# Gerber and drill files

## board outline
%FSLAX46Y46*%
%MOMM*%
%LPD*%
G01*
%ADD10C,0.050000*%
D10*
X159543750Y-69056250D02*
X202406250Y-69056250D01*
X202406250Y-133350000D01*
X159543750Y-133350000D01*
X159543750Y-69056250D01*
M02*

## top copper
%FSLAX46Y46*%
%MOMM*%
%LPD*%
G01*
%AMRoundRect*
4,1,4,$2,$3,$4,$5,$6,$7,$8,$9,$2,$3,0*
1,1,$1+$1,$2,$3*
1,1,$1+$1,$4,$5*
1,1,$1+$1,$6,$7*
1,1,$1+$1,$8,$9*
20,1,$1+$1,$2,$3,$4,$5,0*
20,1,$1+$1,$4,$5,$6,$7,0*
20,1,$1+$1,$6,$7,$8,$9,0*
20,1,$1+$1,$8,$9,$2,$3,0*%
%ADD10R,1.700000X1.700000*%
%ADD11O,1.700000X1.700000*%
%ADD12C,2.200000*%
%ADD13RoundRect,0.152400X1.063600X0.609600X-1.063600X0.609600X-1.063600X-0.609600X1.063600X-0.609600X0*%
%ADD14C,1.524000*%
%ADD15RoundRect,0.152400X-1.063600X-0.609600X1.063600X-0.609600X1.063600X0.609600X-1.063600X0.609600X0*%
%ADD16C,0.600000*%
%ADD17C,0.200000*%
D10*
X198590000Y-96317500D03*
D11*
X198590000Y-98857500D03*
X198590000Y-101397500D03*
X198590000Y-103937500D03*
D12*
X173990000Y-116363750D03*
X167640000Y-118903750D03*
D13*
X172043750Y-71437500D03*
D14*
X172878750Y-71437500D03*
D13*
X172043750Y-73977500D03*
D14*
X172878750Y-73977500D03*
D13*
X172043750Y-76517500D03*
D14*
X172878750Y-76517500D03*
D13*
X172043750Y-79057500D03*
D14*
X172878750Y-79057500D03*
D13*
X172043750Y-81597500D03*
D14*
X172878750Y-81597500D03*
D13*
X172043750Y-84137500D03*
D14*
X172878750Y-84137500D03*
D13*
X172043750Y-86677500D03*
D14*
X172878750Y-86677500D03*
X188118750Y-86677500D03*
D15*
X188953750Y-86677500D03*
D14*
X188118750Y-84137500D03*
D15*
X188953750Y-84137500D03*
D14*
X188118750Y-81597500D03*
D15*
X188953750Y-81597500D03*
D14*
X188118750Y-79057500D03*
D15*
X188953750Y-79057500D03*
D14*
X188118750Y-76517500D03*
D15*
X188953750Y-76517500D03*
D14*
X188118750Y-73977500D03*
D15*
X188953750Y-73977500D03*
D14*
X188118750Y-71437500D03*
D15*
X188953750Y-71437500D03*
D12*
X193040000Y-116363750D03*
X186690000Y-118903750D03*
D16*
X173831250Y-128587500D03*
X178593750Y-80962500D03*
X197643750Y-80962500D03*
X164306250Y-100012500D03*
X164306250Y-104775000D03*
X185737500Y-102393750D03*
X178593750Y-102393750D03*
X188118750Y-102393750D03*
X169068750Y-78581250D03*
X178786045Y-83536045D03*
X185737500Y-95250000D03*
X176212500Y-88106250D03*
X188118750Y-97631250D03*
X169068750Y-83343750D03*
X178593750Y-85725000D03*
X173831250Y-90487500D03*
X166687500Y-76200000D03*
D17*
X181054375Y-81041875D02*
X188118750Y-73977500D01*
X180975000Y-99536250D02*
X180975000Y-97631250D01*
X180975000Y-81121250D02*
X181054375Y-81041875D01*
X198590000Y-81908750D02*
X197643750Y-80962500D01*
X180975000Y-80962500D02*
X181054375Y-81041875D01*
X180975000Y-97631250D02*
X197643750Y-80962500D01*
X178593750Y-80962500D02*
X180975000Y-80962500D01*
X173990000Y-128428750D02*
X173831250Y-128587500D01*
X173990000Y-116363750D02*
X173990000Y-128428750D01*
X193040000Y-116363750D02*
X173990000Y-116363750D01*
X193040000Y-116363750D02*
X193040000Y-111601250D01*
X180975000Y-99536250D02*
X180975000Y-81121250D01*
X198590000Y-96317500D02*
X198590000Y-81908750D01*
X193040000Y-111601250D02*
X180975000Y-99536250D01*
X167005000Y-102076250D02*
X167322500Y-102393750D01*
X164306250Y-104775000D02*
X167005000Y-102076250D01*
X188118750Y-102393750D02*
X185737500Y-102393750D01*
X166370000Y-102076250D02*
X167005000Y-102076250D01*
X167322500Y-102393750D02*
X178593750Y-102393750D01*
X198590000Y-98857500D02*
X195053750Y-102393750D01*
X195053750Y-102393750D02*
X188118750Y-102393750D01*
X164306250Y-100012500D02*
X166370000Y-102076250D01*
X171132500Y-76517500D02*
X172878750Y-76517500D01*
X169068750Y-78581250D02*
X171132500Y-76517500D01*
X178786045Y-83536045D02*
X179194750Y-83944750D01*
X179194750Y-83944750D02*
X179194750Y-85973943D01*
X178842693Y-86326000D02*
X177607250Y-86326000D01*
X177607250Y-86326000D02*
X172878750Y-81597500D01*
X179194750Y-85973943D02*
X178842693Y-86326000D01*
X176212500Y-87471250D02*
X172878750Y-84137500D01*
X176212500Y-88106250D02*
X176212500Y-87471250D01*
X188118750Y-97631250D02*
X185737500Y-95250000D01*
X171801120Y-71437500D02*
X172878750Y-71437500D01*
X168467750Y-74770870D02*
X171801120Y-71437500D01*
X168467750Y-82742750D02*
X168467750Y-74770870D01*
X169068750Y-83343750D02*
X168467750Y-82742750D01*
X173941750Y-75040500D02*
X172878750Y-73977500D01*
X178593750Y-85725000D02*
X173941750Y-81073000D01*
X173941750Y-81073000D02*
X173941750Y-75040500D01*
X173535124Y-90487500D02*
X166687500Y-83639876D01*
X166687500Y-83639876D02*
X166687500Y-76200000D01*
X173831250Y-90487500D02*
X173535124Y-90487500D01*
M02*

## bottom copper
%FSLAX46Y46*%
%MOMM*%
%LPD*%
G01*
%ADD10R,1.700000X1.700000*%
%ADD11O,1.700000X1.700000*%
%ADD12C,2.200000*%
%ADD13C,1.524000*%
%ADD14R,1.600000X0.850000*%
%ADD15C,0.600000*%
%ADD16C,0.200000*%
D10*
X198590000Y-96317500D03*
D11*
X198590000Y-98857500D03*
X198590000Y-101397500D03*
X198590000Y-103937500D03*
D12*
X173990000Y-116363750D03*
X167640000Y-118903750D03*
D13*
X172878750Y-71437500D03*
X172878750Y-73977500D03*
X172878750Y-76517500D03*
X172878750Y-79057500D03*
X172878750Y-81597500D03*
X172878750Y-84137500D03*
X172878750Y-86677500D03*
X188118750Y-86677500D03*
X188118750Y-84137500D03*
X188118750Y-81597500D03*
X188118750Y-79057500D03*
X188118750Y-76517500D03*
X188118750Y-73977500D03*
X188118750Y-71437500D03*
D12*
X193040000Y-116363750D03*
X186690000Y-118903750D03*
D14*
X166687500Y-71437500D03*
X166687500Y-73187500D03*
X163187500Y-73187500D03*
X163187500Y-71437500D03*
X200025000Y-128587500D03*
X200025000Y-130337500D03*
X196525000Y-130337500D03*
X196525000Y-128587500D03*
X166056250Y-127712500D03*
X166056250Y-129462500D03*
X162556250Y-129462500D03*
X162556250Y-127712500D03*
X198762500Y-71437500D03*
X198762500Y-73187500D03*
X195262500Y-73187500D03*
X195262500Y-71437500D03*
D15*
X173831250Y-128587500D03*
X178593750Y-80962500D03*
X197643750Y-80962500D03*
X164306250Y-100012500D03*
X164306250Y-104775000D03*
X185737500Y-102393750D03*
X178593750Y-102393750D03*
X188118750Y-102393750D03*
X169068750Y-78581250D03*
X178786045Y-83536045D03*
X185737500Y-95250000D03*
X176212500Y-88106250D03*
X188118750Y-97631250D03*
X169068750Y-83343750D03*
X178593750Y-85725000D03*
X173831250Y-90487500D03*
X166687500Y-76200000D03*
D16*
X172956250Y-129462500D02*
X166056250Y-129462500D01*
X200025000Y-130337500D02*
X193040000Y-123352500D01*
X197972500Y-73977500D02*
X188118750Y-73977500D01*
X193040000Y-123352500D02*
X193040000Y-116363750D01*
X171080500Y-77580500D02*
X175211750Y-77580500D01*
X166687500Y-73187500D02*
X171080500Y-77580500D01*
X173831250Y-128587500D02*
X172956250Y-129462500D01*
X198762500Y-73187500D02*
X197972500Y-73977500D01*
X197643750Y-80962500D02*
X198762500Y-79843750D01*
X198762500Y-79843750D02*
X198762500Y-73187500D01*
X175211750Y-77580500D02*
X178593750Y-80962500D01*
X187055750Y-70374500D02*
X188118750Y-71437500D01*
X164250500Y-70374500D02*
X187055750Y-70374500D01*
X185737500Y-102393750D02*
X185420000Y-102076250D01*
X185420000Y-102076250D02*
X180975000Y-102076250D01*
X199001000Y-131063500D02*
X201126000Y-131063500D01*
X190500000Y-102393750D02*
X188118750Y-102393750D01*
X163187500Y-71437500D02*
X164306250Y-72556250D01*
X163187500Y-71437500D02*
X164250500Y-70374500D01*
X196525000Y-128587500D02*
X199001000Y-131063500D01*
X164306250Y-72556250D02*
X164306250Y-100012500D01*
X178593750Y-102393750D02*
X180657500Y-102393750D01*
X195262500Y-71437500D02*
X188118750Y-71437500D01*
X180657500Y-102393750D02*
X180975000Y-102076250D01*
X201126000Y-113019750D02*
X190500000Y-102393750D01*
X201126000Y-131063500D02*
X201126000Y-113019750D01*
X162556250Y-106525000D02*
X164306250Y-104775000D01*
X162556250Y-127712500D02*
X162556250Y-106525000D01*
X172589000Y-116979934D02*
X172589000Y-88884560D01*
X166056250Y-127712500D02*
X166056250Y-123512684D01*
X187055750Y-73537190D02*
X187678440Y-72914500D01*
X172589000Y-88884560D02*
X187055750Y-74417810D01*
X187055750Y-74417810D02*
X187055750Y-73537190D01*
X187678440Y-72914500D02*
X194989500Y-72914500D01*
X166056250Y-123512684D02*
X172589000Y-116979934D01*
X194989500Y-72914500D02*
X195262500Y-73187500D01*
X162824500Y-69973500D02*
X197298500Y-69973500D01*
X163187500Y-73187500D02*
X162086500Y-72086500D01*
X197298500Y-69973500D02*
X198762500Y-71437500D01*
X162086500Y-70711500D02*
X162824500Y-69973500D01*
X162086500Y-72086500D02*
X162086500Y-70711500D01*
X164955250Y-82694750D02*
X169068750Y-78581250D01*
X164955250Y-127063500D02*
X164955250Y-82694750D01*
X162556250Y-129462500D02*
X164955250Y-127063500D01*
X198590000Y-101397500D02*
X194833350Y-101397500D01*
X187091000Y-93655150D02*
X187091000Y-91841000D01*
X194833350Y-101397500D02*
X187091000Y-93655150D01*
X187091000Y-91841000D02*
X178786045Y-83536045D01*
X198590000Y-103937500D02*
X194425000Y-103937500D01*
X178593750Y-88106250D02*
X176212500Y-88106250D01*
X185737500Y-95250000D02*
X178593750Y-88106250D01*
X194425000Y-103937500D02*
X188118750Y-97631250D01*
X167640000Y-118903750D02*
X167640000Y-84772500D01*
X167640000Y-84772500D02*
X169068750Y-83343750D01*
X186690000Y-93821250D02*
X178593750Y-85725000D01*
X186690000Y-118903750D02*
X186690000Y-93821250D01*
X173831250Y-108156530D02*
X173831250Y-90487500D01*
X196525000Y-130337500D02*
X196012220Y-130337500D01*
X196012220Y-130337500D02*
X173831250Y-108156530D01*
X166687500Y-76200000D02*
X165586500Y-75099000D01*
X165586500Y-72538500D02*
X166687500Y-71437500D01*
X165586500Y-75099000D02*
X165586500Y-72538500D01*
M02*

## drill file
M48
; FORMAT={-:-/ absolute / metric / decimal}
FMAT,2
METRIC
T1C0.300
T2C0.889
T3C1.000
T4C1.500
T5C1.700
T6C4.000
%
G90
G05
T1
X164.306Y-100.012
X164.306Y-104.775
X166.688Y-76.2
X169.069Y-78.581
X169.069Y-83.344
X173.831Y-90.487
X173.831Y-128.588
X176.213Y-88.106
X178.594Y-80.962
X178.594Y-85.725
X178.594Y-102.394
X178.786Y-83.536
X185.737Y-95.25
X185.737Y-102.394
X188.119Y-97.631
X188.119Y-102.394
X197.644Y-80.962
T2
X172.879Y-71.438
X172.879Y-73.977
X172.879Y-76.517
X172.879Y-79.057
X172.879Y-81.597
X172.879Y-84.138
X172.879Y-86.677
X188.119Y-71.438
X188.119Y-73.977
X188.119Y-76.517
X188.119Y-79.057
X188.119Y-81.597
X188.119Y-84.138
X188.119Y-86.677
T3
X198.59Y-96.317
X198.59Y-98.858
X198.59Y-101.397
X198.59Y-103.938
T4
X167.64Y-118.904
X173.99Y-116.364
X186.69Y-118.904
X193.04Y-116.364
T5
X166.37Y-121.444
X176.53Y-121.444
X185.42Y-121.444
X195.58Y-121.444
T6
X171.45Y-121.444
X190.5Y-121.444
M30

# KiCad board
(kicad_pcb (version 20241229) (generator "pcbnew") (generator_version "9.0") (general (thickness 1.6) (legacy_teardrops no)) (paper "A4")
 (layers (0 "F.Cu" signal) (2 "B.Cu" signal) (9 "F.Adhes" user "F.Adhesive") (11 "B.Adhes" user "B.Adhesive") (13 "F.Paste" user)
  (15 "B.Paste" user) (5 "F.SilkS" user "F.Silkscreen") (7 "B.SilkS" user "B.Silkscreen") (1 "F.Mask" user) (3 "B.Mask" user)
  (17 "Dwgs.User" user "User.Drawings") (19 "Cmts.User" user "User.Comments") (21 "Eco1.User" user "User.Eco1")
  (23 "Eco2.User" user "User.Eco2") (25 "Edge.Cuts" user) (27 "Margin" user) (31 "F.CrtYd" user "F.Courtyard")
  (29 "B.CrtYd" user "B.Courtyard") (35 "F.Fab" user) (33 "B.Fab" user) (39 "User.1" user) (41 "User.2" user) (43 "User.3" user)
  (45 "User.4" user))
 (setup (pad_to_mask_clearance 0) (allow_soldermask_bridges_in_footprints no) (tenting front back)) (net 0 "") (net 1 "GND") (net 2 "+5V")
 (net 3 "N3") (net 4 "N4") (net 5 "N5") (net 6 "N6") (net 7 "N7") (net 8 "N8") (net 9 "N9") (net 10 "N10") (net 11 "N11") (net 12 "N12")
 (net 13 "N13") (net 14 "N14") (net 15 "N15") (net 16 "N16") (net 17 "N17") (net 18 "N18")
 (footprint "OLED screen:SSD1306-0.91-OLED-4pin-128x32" (layer "F.Cu") (at 162.09 94.1275)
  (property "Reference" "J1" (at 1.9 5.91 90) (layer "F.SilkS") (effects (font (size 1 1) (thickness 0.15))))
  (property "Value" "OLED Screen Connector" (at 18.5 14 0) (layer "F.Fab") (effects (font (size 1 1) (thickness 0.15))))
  (pad "1" thru_hole rect (at 36.5 2.19) (size 1.7 1.7) (drill 1) (layers "*.Cu" "*.Mask") (remove_unused_layers no) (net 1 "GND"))
  (pad "2" thru_hole oval (at 36.5 4.73) (size 1.7 1.7) (drill 1) (layers "*.Cu" "*.Mask") (remove_unused_layers no) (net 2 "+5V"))
  (pad "3" thru_hole oval (at 36.5 7.27) (size 1.7 1.7) (drill 1) (layers "*.Cu" "*.Mask") (remove_unused_layers no) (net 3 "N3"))
  (pad "4" thru_hole oval (at 36.5 9.81) (size 1.7 1.7) (drill 1) (layers "*.Cu" "*.Mask") (remove_unused_layers no) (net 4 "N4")))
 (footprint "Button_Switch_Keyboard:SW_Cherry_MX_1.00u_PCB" (layer "F.Cu") (at 173.99 116.36375)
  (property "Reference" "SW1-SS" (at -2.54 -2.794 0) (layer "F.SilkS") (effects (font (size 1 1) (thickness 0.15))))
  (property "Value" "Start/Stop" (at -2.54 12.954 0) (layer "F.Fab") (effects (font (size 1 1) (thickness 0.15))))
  (pad "" np_thru_hole circle (at -7.62 5.08) (size 1.7 1.7) (drill 1.7) (layers "*.Cu" "*.Mask"))
  (pad "" np_thru_hole circle (at -2.54 5.08) (size 4 4) (drill 4) (layers "*.Cu" "*.Mask"))
  (pad "" np_thru_hole circle (at 2.54 5.08) (size 1.7 1.7) (drill 1.7) (layers "*.Cu" "*.Mask"))
  (pad "1" thru_hole circle (at 0 0) (size 2.2 2.2) (drill 1.5) (layers "*.Cu" "*.Mask") (remove_unused_layers no) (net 1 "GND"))
  (pad "2" thru_hole circle (at -6.35 2.54) (size 2.2 2.2) (drill 1.5) (layers "*.Cu" "*.Mask") (remove_unused_layers no) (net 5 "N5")))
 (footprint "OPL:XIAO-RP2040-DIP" (layer "F.Cu") (at 180.49875 79.0575)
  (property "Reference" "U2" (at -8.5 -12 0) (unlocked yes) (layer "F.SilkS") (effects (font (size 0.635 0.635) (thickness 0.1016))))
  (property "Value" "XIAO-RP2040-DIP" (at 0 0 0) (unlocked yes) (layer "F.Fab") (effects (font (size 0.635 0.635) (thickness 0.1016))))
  (pad "1" smd roundrect (at -8.455 -7.62 180) (size 2.432 1.524) (layers "F.Cu" "F.Mask") (roundrect_rratio 0.1) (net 5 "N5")
   (thermal_bridge_angle 45))
  (pad "1" thru_hole circle (at -7.62 -7.62 180) (size 1.524 1.524) (drill 0.889) (layers "*.Cu" "*.Mask") (remove_unused_layers no)
   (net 5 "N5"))
  (pad "2" smd roundrect (at -8.455 -5.08 180) (size 2.432 1.524) (layers "F.Cu" "F.Mask") (roundrect_rratio 0.1) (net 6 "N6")
   (thermal_bridge_angle 45))
  (pad "2" thru_hole circle (at -7.62 -5.08 180) (size 1.524 1.524) (drill 0.889) (layers "*.Cu" "*.Mask") (remove_unused_layers no)
   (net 6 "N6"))
  (pad "3" smd roundrect (at -8.455 -2.54 180) (size 2.432 1.524) (layers "F.Cu" "F.Mask") (roundrect_rratio 0.1) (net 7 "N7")
   (thermal_bridge_angle 45))
  (pad "3" thru_hole circle (at -7.62 -2.54 180) (size 1.524 1.524) (drill 0.889) (layers "*.Cu" "*.Mask") (remove_unused_layers no)
   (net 7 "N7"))
  (pad "4" smd roundrect (at -8.455 0 180) (size 2.432 1.524) (layers "F.Cu" "F.Mask") (roundrect_rratio 0.1) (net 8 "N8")
   (thermal_bridge_angle 45))
  (pad "4" thru_hole circle (at -7.62 0 180) (size 1.524 1.524) (drill 0.889) (layers "*.Cu" "*.Mask") (remove_unused_layers no)
   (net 8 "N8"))
  (pad "5" smd roundrect (at -8.455 2.54 180) (size 2.432 1.524) (layers "F.Cu" "F.Mask") (roundrect_rratio 0.1) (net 3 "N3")
   (thermal_bridge_angle 45))
  (pad "5" thru_hole circle (at -7.62 2.54 180) (size 1.524 1.524) (drill 0.889) (layers "*.Cu" "*.Mask") (remove_unused_layers no)
   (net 3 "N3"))
  (pad "6" smd roundrect (at -8.455 5.08 180) (size 2.432 1.524) (layers "F.Cu" "F.Mask") (roundrect_rratio 0.1) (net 4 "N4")
   (thermal_bridge_angle 45))
  (pad "6" thru_hole circle (at -7.62 5.08 180) (size 1.524 1.524) (drill 0.889) (layers "*.Cu" "*.Mask") (remove_unused_layers no)
   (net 4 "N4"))
  (pad "7" smd roundrect (at -8.455 7.62 180) (size 2.432 1.524) (layers "F.Cu" "F.Mask") (roundrect_rratio 0.1) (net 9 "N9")
   (thermal_bridge_angle 45))
  (pad "7" thru_hole circle (at -7.62 7.62 180) (size 1.524 1.524) (drill 0.889) (layers "*.Cu" "*.Mask") (remove_unused_layers no)
   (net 9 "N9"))
  (pad "8" thru_hole circle (at 7.62 7.62) (size 1.524 1.524) (drill 0.889) (layers "*.Cu" "*.Mask") (remove_unused_layers no)
   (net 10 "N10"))
  (pad "8" smd roundrect (at 8.455 7.62) (size 2.432 1.524) (layers "F.Cu" "F.Mask") (roundrect_rratio 0.1) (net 10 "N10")
   (thermal_bridge_angle 45))
  (pad "9" thru_hole circle (at 7.62 5.08) (size 1.524 1.524) (drill 0.889) (layers "*.Cu" "*.Mask") (remove_unused_layers no)
   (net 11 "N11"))
  (pad "9" smd roundrect (at 8.455 5.08) (size 2.432 1.524) (layers "F.Cu" "F.Mask") (roundrect_rratio 0.1) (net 11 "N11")
   (thermal_bridge_angle 45))
  (pad "10" thru_hole circle (at 7.62 2.54) (size 1.524 1.524) (drill 0.889) (layers "*.Cu" "*.Mask") (remove_unused_layers no)
   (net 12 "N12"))
  (pad "10" smd roundrect (at 8.455 2.54) (size 2.432 1.524) (layers "F.Cu" "F.Mask") (roundrect_rratio 0.1) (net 12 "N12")
   (thermal_bridge_angle 45))
  (pad "11" thru_hole circle (at 7.62 0) (size 1.524 1.524) (drill 0.889) (layers "*.Cu" "*.Mask") (remove_unused_layers no) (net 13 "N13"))
  (pad "11" smd roundrect (at 8.455 0) (size 2.432 1.524) (layers "F.Cu" "F.Mask") (roundrect_rratio 0.1) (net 13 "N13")
   (thermal_bridge_angle 45))
  (pad "12" thru_hole circle (at 7.62 -2.54) (size 1.524 1.524) (drill 0.889) (layers "*.Cu" "*.Mask") (remove_unused_layers no)
   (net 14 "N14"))
  (pad "12" smd roundrect (at 8.455 -2.54) (size 2.432 1.524) (layers "F.Cu" "F.Mask") (roundrect_rratio 0.1) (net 14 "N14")
   (thermal_bridge_angle 45))
  (pad "13" thru_hole circle (at 7.62 -5.08) (size 1.524 1.524) (drill 0.889) (layers "*.Cu" "*.Mask") (remove_unused_layers no)
   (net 1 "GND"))
  (pad "13" smd roundrect (at 8.455 -5.08) (size 2.432 1.524) (layers "F.Cu" "F.Mask") (roundrect_rratio 0.1) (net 1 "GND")
   (thermal_bridge_angle 45))
  (pad "14" thru_hole circle (at 7.62 -7.62) (size 1.524 1.524) (drill 0.889) (layers "*.Cu" "*.Mask") (remove_unused_layers no)
   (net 2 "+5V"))
  (pad "14" smd roundrect (at 8.455 -7.62) (size 2.432 1.524) (layers "F.Cu" "F.Mask") (roundrect_rratio 0.1) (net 2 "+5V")
   (thermal_bridge_angle 45)))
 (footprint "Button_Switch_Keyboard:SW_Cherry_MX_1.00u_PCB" (layer "F.Cu") (at 193.04 116.36375)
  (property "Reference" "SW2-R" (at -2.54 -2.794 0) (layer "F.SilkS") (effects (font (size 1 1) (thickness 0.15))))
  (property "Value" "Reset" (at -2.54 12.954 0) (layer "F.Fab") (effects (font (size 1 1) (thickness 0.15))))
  (pad "" np_thru_hole circle (at -7.62 5.08) (size 1.7 1.7) (drill 1.7) (layers "*.Cu" "*.Mask"))
  (pad "" np_thru_hole circle (at -2.54 5.08) (size 4 4) (drill 4) (layers "*.Cu" "*.Mask"))
  (pad "" np_thru_hole circle (at 2.54 5.08) (size 1.7 1.7) (drill 1.7) (layers "*.Cu" "*.Mask"))
  (pad "1" thru_hole circle (at 0 0) (size 2.2 2.2) (drill 1.5) (layers "*.Cu" "*.Mask") (remove_unused_layers no) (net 1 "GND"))
  (pad "2" thru_hole circle (at -6.35 2.54) (size 2.2 2.2) (drill 1.5) (layers "*.Cu" "*.Mask") (remove_unused_layers no) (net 6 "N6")))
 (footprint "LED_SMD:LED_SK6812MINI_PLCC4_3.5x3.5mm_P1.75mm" (layer "B.Cu") (at 164.9375 72.3125 180)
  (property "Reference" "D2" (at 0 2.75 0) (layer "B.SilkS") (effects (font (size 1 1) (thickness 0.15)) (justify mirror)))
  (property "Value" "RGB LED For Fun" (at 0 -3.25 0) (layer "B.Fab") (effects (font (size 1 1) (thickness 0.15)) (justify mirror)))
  (pad "1" smd rect (at -1.75 0.875 180) (size 1.6 0.85) (layers "B.Cu" "B.Mask" "B.Paste") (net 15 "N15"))
  (pad "2" smd rect (at -1.75 -0.875 180) (size 1.6 0.85) (layers "B.Cu" "B.Mask" "B.Paste") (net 1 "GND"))
  (pad "3" smd rect (at 1.75 -0.875 180) (size 1.6 0.85) (layers "B.Cu" "B.Mask" "B.Paste") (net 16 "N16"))
  (pad "4" smd rect (at 1.75 0.875 180) (size 1.6 0.85) (layers "B.Cu" "B.Mask" "B.Paste") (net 2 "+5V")))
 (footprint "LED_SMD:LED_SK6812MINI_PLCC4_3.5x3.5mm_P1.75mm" (layer "B.Cu") (at 198.275 129.4625 180)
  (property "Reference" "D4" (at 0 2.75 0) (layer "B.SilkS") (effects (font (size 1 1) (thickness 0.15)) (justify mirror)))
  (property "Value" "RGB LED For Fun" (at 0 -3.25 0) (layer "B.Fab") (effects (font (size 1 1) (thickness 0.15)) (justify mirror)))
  (pad "1" smd rect (at -1.75 0.875 180) (size 1.6 0.85) (layers "B.Cu" "B.Mask" "B.Paste") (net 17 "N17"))
  (pad "2" smd rect (at -1.75 -0.875 180) (size 1.6 0.85) (layers "B.Cu" "B.Mask" "B.Paste") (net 1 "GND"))
  (pad "3" smd rect (at 1.75 -0.875 180) (size 1.6 0.85) (layers "B.Cu" "B.Mask" "B.Paste") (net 15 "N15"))
  (pad "4" smd rect (at 1.75 0.875 180) (size 1.6 0.85) (layers "B.Cu" "B.Mask" "B.Paste") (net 2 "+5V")))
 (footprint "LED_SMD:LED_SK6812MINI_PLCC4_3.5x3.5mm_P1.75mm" (layer "B.Cu") (at 164.30625 128.5875 180)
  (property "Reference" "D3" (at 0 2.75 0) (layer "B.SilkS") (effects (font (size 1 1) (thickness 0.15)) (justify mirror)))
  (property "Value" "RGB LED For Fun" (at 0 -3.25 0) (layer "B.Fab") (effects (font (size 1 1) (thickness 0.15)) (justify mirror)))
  (pad "1" smd rect (at -1.75 0.875 180) (size 1.6 0.85) (layers "B.Cu" "B.Mask" "B.Paste") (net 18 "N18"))
  (pad "2" smd rect (at -1.75 -0.875 180) (size 1.6 0.85) (layers "B.Cu" "B.Mask" "B.Paste") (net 1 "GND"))
  (pad "3" smd rect (at 1.75 -0.875 180) (size 1.6 0.85) (layers "B.Cu" "B.Mask" "B.Paste") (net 7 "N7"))
  (pad "4" smd rect (at 1.75 0.875 180) (size 1.6 0.85) (layers "B.Cu" "B.Mask" "B.Paste") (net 2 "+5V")))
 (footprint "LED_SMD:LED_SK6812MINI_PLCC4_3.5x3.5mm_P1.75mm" (layer "B.Cu") (at 197.0125 72.3125 180)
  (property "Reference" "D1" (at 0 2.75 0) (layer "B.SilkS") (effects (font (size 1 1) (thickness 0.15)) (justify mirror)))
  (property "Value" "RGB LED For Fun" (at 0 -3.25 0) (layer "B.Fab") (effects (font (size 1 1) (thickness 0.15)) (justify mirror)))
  (pad "1" smd rect (at -1.75 0.875 180) (size 1.6 0.85) (layers "B.Cu" "B.Mask" "B.Paste") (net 16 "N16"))
  (pad "2" smd rect (at -1.75 -0.875 180) (size 1.6 0.85) (layers "B.Cu" "B.Mask" "B.Paste") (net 1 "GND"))
  (pad "3" smd rect (at 1.75 -0.875 180) (size 1.6 0.85) (layers "B.Cu" "B.Mask" "B.Paste") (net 18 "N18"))
  (pad "4" smd rect (at 1.75 0.875 180) (size 1.6 0.85) (layers "B.Cu" "B.Mask" "B.Paste") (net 2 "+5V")))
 (gr_rect (start 159.54375 69.05625) (end 202.40625 133.35) (stroke (width 0.05) (type default)) (fill no) (layer "Edge.Cuts"))
 (segment (start 181.054375 81.041875) (end 188.11875 73.9775) (width 0.2) (layer "F.Cu") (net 1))
 (segment (start 180.975 99.53625) (end 180.975 97.63125) (width 0.2) (layer "F.Cu") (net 1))
 (segment (start 180.975 81.12125) (end 181.054375 81.041875) (width 0.2) (layer "F.Cu") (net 1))
 (segment (start 198.59 81.90875) (end 197.64375 80.9625) (width 0.2) (layer "F.Cu") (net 1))
 (segment (start 180.975 80.9625) (end 181.054375 81.041875) (width 0.2) (layer "F.Cu") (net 1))
 (segment (start 180.975 97.63125) (end 197.64375 80.9625) (width 0.2) (layer "F.Cu") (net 1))
 (segment (start 178.59375 80.9625) (end 180.975 80.9625) (width 0.2) (layer "F.Cu") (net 1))
 (segment (start 173.99 128.42875) (end 173.83125 128.5875) (width 0.2) (layer "F.Cu") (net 1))
 (segment (start 173.99 116.36375) (end 173.99 128.42875) (width 0.2) (layer "F.Cu") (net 1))
 (segment (start 193.04 116.36375) (end 173.99 116.36375) (width 0.2) (layer "F.Cu") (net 1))
 (segment (start 193.04 116.36375) (end 193.04 111.60125) (width 0.2) (layer "F.Cu") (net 1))
 (segment (start 180.975 99.53625) (end 180.975 81.12125) (width 0.2) (layer "F.Cu") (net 1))
 (segment (start 198.59 96.3175) (end 198.59 81.90875) (width 0.2) (layer "F.Cu") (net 1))
 (segment (start 193.04 111.60125) (end 180.975 99.53625) (width 0.2) (layer "F.Cu") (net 1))
 (via (at 173.83125 128.5875) (size 0.6) (drill 0.3) (layers "F.Cu" "B.Cu") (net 1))
 (via (at 178.59375 80.9625) (size 0.6) (drill 0.3) (layers "F.Cu" "B.Cu") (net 1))
 (via (at 197.64375 80.9625) (size 0.6) (drill 0.3) (layers "F.Cu" "B.Cu") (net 1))
 (segment (start 172.95625 129.4625) (end 166.05625 129.4625) (width 0.2) (layer "B.Cu") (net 1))
 (segment (start 200.025 130.3375) (end 193.04 123.3525) (width 0.2) (layer "B.Cu") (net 1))
 (segment (start 197.9725 73.9775) (end 188.11875 73.9775) (width 0.2) (layer "B.Cu") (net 1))
 (segment (start 193.04 123.3525) (end 193.04 116.36375) (width 0.2) (layer "B.Cu") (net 1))
 (segment (start 171.0805 77.5805) (end 175.21175 77.5805) (width 0.2) (layer "B.Cu") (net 1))
 (segment (start 166.6875 73.1875) (end 171.0805 77.5805) (width 0.2) (layer "B.Cu") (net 1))
 (segment (start 173.83125 128.5875) (end 172.95625 129.4625) (width 0.2) (layer "B.Cu") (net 1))
 (segment (start 198.7625 73.1875) (end 197.9725 73.9775) (width 0.2) (layer "B.Cu") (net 1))
 (segment (start 197.64375 80.9625) (end 198.7625 79.84375) (width 0.2) (layer "B.Cu") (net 1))
 (segment (start 198.7625 79.84375) (end 198.7625 73.1875) (width 0.2) (layer "B.Cu") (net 1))
 (segment (start 175.21175 77.5805) (end 178.59375 80.9625) (width 0.2) (layer "B.Cu") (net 1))
 (segment (start 167.005 102.07625) (end 167.3225 102.39375) (width 0.2) (layer "F.Cu") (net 2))
 (segment (start 164.30625 104.775) (end 167.005 102.07625) (width 0.2) (layer "F.Cu") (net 2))
 (segment (start 188.11875 102.39375) (end 185.7375 102.39375) (width 0.2) (layer "F.Cu") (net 2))
 (segment (start 166.37 102.07625) (end 167.005 102.07625) (width 0.2) (layer "F.Cu") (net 2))
 (segment (start 167.3225 102.39375) (end 178.59375 102.39375) (width 0.2) (layer "F.Cu") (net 2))
 (segment (start 198.59 98.8575) (end 195.05375 102.39375) (width 0.2) (layer "F.Cu") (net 2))
 (segment (start 195.05375 102.39375) (end 188.11875 102.39375) (width 0.2) (layer "F.Cu") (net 2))
 (segment (start 164.30625 100.0125) (end 166.37 102.07625) (width 0.2) (layer "F.Cu") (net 2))
 (via (at 164.30625 100.0125) (size 0.6) (drill 0.3) (layers "F.Cu" "B.Cu") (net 2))
 (via (at 164.30625 104.775) (size 0.6) (drill 0.3) (layers "F.Cu" "B.Cu") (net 2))
 (via (at 185.7375 102.39375) (size 0.6) (drill 0.3) (layers "F.Cu" "B.Cu") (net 2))
 (via (at 178.59375 102.39375) (size 0.6) (drill 0.3) (layers "F.Cu" "B.Cu") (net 2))
 (via (at 188.11875 102.39375) (size 0.6) (drill 0.3) (layers "F.Cu" "B.Cu") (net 2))
 (segment (start 187.05575 70.3745) (end 188.11875 71.4375) (width 0.2) (layer "B.Cu") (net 2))
 (segment (start 164.2505 70.3745) (end 187.05575 70.3745) (width 0.2) (layer "B.Cu") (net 2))
 (segment (start 185.7375 102.39375) (end 185.42 102.07625) (width 0.2) (layer "B.Cu") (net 2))
 (segment (start 185.42 102.07625) (end 180.975 102.07625) (width 0.2) (layer "B.Cu") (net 2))
 (segment (start 199.001 131.0635) (end 201.126 131.0635) (width 0.2) (layer "B.Cu") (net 2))
 (segment (start 190.5 102.39375) (end 188.11875 102.39375) (width 0.2) (layer "B.Cu") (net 2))
 (segment (start 163.1875 71.4375) (end 164.30625 72.55625) (width 0.2) (layer "B.Cu") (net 2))
 (segment (start 163.1875 71.4375) (end 164.2505 70.3745) (width 0.2) (layer "B.Cu") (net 2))
 (segment (start 196.525 128.5875) (end 199.001 131.0635) (width 0.2) (layer "B.Cu") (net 2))
 (segment (start 164.30625 72.55625) (end 164.30625 100.0125) (width 0.2) (layer "B.Cu") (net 2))
 (segment (start 178.59375 102.39375) (end 180.6575 102.39375) (width 0.2) (layer "B.Cu") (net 2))
 (segment (start 195.2625 71.4375) (end 188.11875 71.4375) (width 0.2) (layer "B.Cu") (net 2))
 (segment (start 180.6575 102.39375) (end 180.975 102.07625) (width 0.2) (layer "B.Cu") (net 2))
 (segment (start 201.126 113.01975) (end 190.5 102.39375) (width 0.2) (layer "B.Cu") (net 2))
 (segment (start 201.126 131.0635) (end 201.126 113.01975) (width 0.2) (layer "B.Cu") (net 2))
 (segment (start 162.55625 106.525) (end 164.30625 104.775) (width 0.2) (layer "B.Cu") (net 2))
 (segment (start 162.55625 127.7125) (end 162.55625 106.525) (width 0.2) (layer "B.Cu") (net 2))
 (segment (start 172.589 116.979934) (end 172.589 88.88456) (width 0.2) (layer "B.Cu") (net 18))
 (segment (start 166.05625 127.7125) (end 166.05625 123.512684) (width 0.2) (layer "B.Cu") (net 18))
 (segment (start 187.05575 73.53719) (end 187.67844 72.9145) (width 0.2) (layer "B.Cu") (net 18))
 (segment (start 172.589 88.88456) (end 187.05575 74.41781) (width 0.2) (layer "B.Cu") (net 18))
 (segment (start 187.05575 74.41781) (end 187.05575 73.53719) (width 0.2) (layer "B.Cu") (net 18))
 (segment (start 187.67844 72.9145) (end 194.9895 72.9145) (width 0.2) (layer "B.Cu") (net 18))
 (segment (start 166.05625 123.512684) (end 172.589 116.979934) (width 0.2) (layer "B.Cu") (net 18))
 (segment (start 194.9895 72.9145) (end 195.2625 73.1875) (width 0.2) (layer "B.Cu") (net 18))
 (segment (start 162.8245 69.9735) (end 197.2985 69.9735) (width 0.2) (layer "B.Cu") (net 16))
 (segment (start 163.1875 73.1875) (end 162.0865 72.0865) (width 0.2) (layer "B.Cu") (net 16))
 (segment (start 197.2985 69.9735) (end 198.7625 71.4375) (width 0.2) (layer "B.Cu") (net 16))
 (segment (start 162.0865 70.7115) (end 162.8245 69.9735) (width 0.2) (layer "B.Cu") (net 16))
 (segment (start 162.0865 72.0865) (end 162.0865 70.7115) (width 0.2) (layer "B.Cu") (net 16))
 (segment (start 171.1325 76.5175) (end 172.87875 76.5175) (width 0.2) (layer "F.Cu") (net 7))
 (segment (start 169.06875 78.58125) (end 171.1325 76.5175) (width 0.2) (layer "F.Cu") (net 7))
 (via (at 169.06875 78.58125) (size 0.6) (drill 0.3) (layers "F.Cu" "B.Cu") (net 7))
 (segment (start 164.95525 82.69475) (end 169.06875 78.58125) (width 0.2) (layer "B.Cu") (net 7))
 (segment (start 164.95525 127.0635) (end 164.95525 82.69475) (width 0.2) (layer "B.Cu") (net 7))
 (segment (start 162.55625 129.4625) (end 164.95525 127.0635) (width 0.2) (layer "B.Cu") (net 7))
 (segment (start 178.786045 83.536045) (end 179.19475 83.94475) (width 0.2) (layer "F.Cu") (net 3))
 (segment (start 179.19475 83.94475) (end 179.19475 85.973943) (width 0.2) (layer "F.Cu") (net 3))
 (segment (start 178.842693 86.326) (end 177.60725 86.326) (width 0.2) (layer "F.Cu") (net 3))
 (segment (start 177.60725 86.326) (end 172.87875 81.5975) (width 0.2) (layer "F.Cu") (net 3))
 (segment (start 179.19475 85.973943) (end 178.842693 86.326) (width 0.2) (layer "F.Cu") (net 3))
 (via (at 178.786045 83.536045) (size 0.6) (drill 0.3) (layers "F.Cu" "B.Cu") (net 3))
 (segment (start 198.59 101.3975) (end 194.83335 101.3975) (width 0.2) (layer "B.Cu") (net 3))
 (segment (start 187.091 93.65515) (end 187.091 91.841) (width 0.2) (layer "B.Cu") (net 3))
 (segment (start 194.83335 101.3975) (end 187.091 93.65515) (width 0.2) (layer "B.Cu") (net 3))
 (segment (start 187.091 91.841) (end 178.786045 83.536045) (width 0.2) (layer "B.Cu") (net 3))
 (segment (start 176.2125 87.47125) (end 172.87875 84.1375) (width 0.2) (layer "F.Cu") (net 4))
 (segment (start 176.2125 88.10625) (end 176.2125 87.47125) (width 0.2) (layer "F.Cu") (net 4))
 (segment (start 188.11875 97.63125) (end 185.7375 95.25) (width 0.2) (layer "F.Cu") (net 4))
 (via (at 185.7375 95.25) (size 0.6) (drill 0.3) (layers "F.Cu" "B.Cu") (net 4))
 (via (at 176.2125 88.10625) (size 0.6) (drill 0.3) (layers "F.Cu" "B.Cu") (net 4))
 (via (at 188.11875 97.63125) (size 0.6) (drill 0.3) (layers "F.Cu" "B.Cu") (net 4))
 (segment (start 198.59 103.9375) (end 194.425 103.9375) (width 0.2) (layer "B.Cu") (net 4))
 (segment (start 178.59375 88.10625) (end 176.2125 88.10625) (width 0.2) (layer "B.Cu") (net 4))
 (segment (start 185.7375 95.25) (end 178.59375 88.10625) (width 0.2) (layer "B.Cu") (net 4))
 (segment (start 194.425 103.9375) (end 188.11875 97.63125) (width 0.2) (layer "B.Cu") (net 4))
 (segment (start 171.80112 71.4375) (end 172.87875 71.4375) (width 0.2) (layer "F.Cu") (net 5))
 (segment (start 168.46775 74.77087) (end 171.80112 71.4375) (width 0.2) (layer "F.Cu") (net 5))
 (segment (start 168.46775 82.74275) (end 168.46775 74.77087) (width 0.2) (layer "F.Cu") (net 5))
 (segment (start 169.06875 83.34375) (end 168.46775 82.74275) (width 0.2) (layer "F.Cu") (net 5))
 (via (at 169.06875 83.34375) (size 0.6) (drill 0.3) (layers "F.Cu" "B.Cu") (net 5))
 (segment (start 167.64 118.90375) (end 167.64 84.7725) (width 0.2) (layer "B.Cu") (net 5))
 (segment (start 167.64 84.7725) (end 169.06875 83.34375) (width 0.2) (layer "B.Cu") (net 5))
 (segment (start 173.94175 75.0405) (end 172.87875 73.9775) (width 0.2) (layer "F.Cu") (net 6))
 (segment (start 178.59375 85.725) (end 173.94175 81.073) (width 0.2) (layer "F.Cu") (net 6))
 (segment (start 173.94175 81.073) (end 173.94175 75.0405) (width 0.2) (layer "F.Cu") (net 6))
 (via (at 178.59375 85.725) (size 0.6) (drill 0.3) (layers "F.Cu" "B.Cu") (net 6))
 (segment (start 186.69 93.82125) (end 178.59375 85.725) (width 0.2) (layer "B.Cu") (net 6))
 (segment (start 186.69 118.90375) (end 186.69 93.82125) (width 0.2) (layer "B.Cu") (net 6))
 (segment (start 173.535124 90.4875) (end 166.6875 83.639876) (width 0.2) (layer "F.Cu") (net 15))
 (segment (start 166.6875 83.639876) (end 166.6875 76.2) (width 0.2) (layer "F.Cu") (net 15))
 (segment (start 173.83125 90.4875) (end 173.535124 90.4875) (width 0.2) (layer "F.Cu") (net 15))
 (via (at 173.83125 90.4875) (size 0.6) (drill 0.3) (layers "F.Cu" "B.Cu") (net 15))
 (via (at 166.6875 76.2) (size 0.6) (drill 0.3) (layers "F.Cu" "B.Cu") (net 15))
 (segment (start 173.83125 108.15653) (end 173.83125 90.4875) (width 0.2) (layer "B.Cu") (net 15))
 (segment (start 196.525 130.3375) (end 196.01222 130.3375) (width 0.2) (layer "B.Cu") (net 15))
 (segment (start 196.01222 130.3375) (end 173.83125 108.15653) (width 0.2) (layer "B.Cu") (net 15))
 (segment (start 166.6875 76.2) (end 165.5865 75.099) (width 0.2) (layer "B.Cu") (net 15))
 (segment (start 165.5865 72.5385) (end 166.6875 71.4375) (width 0.2) (layer "B.Cu") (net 15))
 (segment (start 165.5865 75.099) (end 165.5865 72.5385) (width 0.2) (layer "B.Cu") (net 15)))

